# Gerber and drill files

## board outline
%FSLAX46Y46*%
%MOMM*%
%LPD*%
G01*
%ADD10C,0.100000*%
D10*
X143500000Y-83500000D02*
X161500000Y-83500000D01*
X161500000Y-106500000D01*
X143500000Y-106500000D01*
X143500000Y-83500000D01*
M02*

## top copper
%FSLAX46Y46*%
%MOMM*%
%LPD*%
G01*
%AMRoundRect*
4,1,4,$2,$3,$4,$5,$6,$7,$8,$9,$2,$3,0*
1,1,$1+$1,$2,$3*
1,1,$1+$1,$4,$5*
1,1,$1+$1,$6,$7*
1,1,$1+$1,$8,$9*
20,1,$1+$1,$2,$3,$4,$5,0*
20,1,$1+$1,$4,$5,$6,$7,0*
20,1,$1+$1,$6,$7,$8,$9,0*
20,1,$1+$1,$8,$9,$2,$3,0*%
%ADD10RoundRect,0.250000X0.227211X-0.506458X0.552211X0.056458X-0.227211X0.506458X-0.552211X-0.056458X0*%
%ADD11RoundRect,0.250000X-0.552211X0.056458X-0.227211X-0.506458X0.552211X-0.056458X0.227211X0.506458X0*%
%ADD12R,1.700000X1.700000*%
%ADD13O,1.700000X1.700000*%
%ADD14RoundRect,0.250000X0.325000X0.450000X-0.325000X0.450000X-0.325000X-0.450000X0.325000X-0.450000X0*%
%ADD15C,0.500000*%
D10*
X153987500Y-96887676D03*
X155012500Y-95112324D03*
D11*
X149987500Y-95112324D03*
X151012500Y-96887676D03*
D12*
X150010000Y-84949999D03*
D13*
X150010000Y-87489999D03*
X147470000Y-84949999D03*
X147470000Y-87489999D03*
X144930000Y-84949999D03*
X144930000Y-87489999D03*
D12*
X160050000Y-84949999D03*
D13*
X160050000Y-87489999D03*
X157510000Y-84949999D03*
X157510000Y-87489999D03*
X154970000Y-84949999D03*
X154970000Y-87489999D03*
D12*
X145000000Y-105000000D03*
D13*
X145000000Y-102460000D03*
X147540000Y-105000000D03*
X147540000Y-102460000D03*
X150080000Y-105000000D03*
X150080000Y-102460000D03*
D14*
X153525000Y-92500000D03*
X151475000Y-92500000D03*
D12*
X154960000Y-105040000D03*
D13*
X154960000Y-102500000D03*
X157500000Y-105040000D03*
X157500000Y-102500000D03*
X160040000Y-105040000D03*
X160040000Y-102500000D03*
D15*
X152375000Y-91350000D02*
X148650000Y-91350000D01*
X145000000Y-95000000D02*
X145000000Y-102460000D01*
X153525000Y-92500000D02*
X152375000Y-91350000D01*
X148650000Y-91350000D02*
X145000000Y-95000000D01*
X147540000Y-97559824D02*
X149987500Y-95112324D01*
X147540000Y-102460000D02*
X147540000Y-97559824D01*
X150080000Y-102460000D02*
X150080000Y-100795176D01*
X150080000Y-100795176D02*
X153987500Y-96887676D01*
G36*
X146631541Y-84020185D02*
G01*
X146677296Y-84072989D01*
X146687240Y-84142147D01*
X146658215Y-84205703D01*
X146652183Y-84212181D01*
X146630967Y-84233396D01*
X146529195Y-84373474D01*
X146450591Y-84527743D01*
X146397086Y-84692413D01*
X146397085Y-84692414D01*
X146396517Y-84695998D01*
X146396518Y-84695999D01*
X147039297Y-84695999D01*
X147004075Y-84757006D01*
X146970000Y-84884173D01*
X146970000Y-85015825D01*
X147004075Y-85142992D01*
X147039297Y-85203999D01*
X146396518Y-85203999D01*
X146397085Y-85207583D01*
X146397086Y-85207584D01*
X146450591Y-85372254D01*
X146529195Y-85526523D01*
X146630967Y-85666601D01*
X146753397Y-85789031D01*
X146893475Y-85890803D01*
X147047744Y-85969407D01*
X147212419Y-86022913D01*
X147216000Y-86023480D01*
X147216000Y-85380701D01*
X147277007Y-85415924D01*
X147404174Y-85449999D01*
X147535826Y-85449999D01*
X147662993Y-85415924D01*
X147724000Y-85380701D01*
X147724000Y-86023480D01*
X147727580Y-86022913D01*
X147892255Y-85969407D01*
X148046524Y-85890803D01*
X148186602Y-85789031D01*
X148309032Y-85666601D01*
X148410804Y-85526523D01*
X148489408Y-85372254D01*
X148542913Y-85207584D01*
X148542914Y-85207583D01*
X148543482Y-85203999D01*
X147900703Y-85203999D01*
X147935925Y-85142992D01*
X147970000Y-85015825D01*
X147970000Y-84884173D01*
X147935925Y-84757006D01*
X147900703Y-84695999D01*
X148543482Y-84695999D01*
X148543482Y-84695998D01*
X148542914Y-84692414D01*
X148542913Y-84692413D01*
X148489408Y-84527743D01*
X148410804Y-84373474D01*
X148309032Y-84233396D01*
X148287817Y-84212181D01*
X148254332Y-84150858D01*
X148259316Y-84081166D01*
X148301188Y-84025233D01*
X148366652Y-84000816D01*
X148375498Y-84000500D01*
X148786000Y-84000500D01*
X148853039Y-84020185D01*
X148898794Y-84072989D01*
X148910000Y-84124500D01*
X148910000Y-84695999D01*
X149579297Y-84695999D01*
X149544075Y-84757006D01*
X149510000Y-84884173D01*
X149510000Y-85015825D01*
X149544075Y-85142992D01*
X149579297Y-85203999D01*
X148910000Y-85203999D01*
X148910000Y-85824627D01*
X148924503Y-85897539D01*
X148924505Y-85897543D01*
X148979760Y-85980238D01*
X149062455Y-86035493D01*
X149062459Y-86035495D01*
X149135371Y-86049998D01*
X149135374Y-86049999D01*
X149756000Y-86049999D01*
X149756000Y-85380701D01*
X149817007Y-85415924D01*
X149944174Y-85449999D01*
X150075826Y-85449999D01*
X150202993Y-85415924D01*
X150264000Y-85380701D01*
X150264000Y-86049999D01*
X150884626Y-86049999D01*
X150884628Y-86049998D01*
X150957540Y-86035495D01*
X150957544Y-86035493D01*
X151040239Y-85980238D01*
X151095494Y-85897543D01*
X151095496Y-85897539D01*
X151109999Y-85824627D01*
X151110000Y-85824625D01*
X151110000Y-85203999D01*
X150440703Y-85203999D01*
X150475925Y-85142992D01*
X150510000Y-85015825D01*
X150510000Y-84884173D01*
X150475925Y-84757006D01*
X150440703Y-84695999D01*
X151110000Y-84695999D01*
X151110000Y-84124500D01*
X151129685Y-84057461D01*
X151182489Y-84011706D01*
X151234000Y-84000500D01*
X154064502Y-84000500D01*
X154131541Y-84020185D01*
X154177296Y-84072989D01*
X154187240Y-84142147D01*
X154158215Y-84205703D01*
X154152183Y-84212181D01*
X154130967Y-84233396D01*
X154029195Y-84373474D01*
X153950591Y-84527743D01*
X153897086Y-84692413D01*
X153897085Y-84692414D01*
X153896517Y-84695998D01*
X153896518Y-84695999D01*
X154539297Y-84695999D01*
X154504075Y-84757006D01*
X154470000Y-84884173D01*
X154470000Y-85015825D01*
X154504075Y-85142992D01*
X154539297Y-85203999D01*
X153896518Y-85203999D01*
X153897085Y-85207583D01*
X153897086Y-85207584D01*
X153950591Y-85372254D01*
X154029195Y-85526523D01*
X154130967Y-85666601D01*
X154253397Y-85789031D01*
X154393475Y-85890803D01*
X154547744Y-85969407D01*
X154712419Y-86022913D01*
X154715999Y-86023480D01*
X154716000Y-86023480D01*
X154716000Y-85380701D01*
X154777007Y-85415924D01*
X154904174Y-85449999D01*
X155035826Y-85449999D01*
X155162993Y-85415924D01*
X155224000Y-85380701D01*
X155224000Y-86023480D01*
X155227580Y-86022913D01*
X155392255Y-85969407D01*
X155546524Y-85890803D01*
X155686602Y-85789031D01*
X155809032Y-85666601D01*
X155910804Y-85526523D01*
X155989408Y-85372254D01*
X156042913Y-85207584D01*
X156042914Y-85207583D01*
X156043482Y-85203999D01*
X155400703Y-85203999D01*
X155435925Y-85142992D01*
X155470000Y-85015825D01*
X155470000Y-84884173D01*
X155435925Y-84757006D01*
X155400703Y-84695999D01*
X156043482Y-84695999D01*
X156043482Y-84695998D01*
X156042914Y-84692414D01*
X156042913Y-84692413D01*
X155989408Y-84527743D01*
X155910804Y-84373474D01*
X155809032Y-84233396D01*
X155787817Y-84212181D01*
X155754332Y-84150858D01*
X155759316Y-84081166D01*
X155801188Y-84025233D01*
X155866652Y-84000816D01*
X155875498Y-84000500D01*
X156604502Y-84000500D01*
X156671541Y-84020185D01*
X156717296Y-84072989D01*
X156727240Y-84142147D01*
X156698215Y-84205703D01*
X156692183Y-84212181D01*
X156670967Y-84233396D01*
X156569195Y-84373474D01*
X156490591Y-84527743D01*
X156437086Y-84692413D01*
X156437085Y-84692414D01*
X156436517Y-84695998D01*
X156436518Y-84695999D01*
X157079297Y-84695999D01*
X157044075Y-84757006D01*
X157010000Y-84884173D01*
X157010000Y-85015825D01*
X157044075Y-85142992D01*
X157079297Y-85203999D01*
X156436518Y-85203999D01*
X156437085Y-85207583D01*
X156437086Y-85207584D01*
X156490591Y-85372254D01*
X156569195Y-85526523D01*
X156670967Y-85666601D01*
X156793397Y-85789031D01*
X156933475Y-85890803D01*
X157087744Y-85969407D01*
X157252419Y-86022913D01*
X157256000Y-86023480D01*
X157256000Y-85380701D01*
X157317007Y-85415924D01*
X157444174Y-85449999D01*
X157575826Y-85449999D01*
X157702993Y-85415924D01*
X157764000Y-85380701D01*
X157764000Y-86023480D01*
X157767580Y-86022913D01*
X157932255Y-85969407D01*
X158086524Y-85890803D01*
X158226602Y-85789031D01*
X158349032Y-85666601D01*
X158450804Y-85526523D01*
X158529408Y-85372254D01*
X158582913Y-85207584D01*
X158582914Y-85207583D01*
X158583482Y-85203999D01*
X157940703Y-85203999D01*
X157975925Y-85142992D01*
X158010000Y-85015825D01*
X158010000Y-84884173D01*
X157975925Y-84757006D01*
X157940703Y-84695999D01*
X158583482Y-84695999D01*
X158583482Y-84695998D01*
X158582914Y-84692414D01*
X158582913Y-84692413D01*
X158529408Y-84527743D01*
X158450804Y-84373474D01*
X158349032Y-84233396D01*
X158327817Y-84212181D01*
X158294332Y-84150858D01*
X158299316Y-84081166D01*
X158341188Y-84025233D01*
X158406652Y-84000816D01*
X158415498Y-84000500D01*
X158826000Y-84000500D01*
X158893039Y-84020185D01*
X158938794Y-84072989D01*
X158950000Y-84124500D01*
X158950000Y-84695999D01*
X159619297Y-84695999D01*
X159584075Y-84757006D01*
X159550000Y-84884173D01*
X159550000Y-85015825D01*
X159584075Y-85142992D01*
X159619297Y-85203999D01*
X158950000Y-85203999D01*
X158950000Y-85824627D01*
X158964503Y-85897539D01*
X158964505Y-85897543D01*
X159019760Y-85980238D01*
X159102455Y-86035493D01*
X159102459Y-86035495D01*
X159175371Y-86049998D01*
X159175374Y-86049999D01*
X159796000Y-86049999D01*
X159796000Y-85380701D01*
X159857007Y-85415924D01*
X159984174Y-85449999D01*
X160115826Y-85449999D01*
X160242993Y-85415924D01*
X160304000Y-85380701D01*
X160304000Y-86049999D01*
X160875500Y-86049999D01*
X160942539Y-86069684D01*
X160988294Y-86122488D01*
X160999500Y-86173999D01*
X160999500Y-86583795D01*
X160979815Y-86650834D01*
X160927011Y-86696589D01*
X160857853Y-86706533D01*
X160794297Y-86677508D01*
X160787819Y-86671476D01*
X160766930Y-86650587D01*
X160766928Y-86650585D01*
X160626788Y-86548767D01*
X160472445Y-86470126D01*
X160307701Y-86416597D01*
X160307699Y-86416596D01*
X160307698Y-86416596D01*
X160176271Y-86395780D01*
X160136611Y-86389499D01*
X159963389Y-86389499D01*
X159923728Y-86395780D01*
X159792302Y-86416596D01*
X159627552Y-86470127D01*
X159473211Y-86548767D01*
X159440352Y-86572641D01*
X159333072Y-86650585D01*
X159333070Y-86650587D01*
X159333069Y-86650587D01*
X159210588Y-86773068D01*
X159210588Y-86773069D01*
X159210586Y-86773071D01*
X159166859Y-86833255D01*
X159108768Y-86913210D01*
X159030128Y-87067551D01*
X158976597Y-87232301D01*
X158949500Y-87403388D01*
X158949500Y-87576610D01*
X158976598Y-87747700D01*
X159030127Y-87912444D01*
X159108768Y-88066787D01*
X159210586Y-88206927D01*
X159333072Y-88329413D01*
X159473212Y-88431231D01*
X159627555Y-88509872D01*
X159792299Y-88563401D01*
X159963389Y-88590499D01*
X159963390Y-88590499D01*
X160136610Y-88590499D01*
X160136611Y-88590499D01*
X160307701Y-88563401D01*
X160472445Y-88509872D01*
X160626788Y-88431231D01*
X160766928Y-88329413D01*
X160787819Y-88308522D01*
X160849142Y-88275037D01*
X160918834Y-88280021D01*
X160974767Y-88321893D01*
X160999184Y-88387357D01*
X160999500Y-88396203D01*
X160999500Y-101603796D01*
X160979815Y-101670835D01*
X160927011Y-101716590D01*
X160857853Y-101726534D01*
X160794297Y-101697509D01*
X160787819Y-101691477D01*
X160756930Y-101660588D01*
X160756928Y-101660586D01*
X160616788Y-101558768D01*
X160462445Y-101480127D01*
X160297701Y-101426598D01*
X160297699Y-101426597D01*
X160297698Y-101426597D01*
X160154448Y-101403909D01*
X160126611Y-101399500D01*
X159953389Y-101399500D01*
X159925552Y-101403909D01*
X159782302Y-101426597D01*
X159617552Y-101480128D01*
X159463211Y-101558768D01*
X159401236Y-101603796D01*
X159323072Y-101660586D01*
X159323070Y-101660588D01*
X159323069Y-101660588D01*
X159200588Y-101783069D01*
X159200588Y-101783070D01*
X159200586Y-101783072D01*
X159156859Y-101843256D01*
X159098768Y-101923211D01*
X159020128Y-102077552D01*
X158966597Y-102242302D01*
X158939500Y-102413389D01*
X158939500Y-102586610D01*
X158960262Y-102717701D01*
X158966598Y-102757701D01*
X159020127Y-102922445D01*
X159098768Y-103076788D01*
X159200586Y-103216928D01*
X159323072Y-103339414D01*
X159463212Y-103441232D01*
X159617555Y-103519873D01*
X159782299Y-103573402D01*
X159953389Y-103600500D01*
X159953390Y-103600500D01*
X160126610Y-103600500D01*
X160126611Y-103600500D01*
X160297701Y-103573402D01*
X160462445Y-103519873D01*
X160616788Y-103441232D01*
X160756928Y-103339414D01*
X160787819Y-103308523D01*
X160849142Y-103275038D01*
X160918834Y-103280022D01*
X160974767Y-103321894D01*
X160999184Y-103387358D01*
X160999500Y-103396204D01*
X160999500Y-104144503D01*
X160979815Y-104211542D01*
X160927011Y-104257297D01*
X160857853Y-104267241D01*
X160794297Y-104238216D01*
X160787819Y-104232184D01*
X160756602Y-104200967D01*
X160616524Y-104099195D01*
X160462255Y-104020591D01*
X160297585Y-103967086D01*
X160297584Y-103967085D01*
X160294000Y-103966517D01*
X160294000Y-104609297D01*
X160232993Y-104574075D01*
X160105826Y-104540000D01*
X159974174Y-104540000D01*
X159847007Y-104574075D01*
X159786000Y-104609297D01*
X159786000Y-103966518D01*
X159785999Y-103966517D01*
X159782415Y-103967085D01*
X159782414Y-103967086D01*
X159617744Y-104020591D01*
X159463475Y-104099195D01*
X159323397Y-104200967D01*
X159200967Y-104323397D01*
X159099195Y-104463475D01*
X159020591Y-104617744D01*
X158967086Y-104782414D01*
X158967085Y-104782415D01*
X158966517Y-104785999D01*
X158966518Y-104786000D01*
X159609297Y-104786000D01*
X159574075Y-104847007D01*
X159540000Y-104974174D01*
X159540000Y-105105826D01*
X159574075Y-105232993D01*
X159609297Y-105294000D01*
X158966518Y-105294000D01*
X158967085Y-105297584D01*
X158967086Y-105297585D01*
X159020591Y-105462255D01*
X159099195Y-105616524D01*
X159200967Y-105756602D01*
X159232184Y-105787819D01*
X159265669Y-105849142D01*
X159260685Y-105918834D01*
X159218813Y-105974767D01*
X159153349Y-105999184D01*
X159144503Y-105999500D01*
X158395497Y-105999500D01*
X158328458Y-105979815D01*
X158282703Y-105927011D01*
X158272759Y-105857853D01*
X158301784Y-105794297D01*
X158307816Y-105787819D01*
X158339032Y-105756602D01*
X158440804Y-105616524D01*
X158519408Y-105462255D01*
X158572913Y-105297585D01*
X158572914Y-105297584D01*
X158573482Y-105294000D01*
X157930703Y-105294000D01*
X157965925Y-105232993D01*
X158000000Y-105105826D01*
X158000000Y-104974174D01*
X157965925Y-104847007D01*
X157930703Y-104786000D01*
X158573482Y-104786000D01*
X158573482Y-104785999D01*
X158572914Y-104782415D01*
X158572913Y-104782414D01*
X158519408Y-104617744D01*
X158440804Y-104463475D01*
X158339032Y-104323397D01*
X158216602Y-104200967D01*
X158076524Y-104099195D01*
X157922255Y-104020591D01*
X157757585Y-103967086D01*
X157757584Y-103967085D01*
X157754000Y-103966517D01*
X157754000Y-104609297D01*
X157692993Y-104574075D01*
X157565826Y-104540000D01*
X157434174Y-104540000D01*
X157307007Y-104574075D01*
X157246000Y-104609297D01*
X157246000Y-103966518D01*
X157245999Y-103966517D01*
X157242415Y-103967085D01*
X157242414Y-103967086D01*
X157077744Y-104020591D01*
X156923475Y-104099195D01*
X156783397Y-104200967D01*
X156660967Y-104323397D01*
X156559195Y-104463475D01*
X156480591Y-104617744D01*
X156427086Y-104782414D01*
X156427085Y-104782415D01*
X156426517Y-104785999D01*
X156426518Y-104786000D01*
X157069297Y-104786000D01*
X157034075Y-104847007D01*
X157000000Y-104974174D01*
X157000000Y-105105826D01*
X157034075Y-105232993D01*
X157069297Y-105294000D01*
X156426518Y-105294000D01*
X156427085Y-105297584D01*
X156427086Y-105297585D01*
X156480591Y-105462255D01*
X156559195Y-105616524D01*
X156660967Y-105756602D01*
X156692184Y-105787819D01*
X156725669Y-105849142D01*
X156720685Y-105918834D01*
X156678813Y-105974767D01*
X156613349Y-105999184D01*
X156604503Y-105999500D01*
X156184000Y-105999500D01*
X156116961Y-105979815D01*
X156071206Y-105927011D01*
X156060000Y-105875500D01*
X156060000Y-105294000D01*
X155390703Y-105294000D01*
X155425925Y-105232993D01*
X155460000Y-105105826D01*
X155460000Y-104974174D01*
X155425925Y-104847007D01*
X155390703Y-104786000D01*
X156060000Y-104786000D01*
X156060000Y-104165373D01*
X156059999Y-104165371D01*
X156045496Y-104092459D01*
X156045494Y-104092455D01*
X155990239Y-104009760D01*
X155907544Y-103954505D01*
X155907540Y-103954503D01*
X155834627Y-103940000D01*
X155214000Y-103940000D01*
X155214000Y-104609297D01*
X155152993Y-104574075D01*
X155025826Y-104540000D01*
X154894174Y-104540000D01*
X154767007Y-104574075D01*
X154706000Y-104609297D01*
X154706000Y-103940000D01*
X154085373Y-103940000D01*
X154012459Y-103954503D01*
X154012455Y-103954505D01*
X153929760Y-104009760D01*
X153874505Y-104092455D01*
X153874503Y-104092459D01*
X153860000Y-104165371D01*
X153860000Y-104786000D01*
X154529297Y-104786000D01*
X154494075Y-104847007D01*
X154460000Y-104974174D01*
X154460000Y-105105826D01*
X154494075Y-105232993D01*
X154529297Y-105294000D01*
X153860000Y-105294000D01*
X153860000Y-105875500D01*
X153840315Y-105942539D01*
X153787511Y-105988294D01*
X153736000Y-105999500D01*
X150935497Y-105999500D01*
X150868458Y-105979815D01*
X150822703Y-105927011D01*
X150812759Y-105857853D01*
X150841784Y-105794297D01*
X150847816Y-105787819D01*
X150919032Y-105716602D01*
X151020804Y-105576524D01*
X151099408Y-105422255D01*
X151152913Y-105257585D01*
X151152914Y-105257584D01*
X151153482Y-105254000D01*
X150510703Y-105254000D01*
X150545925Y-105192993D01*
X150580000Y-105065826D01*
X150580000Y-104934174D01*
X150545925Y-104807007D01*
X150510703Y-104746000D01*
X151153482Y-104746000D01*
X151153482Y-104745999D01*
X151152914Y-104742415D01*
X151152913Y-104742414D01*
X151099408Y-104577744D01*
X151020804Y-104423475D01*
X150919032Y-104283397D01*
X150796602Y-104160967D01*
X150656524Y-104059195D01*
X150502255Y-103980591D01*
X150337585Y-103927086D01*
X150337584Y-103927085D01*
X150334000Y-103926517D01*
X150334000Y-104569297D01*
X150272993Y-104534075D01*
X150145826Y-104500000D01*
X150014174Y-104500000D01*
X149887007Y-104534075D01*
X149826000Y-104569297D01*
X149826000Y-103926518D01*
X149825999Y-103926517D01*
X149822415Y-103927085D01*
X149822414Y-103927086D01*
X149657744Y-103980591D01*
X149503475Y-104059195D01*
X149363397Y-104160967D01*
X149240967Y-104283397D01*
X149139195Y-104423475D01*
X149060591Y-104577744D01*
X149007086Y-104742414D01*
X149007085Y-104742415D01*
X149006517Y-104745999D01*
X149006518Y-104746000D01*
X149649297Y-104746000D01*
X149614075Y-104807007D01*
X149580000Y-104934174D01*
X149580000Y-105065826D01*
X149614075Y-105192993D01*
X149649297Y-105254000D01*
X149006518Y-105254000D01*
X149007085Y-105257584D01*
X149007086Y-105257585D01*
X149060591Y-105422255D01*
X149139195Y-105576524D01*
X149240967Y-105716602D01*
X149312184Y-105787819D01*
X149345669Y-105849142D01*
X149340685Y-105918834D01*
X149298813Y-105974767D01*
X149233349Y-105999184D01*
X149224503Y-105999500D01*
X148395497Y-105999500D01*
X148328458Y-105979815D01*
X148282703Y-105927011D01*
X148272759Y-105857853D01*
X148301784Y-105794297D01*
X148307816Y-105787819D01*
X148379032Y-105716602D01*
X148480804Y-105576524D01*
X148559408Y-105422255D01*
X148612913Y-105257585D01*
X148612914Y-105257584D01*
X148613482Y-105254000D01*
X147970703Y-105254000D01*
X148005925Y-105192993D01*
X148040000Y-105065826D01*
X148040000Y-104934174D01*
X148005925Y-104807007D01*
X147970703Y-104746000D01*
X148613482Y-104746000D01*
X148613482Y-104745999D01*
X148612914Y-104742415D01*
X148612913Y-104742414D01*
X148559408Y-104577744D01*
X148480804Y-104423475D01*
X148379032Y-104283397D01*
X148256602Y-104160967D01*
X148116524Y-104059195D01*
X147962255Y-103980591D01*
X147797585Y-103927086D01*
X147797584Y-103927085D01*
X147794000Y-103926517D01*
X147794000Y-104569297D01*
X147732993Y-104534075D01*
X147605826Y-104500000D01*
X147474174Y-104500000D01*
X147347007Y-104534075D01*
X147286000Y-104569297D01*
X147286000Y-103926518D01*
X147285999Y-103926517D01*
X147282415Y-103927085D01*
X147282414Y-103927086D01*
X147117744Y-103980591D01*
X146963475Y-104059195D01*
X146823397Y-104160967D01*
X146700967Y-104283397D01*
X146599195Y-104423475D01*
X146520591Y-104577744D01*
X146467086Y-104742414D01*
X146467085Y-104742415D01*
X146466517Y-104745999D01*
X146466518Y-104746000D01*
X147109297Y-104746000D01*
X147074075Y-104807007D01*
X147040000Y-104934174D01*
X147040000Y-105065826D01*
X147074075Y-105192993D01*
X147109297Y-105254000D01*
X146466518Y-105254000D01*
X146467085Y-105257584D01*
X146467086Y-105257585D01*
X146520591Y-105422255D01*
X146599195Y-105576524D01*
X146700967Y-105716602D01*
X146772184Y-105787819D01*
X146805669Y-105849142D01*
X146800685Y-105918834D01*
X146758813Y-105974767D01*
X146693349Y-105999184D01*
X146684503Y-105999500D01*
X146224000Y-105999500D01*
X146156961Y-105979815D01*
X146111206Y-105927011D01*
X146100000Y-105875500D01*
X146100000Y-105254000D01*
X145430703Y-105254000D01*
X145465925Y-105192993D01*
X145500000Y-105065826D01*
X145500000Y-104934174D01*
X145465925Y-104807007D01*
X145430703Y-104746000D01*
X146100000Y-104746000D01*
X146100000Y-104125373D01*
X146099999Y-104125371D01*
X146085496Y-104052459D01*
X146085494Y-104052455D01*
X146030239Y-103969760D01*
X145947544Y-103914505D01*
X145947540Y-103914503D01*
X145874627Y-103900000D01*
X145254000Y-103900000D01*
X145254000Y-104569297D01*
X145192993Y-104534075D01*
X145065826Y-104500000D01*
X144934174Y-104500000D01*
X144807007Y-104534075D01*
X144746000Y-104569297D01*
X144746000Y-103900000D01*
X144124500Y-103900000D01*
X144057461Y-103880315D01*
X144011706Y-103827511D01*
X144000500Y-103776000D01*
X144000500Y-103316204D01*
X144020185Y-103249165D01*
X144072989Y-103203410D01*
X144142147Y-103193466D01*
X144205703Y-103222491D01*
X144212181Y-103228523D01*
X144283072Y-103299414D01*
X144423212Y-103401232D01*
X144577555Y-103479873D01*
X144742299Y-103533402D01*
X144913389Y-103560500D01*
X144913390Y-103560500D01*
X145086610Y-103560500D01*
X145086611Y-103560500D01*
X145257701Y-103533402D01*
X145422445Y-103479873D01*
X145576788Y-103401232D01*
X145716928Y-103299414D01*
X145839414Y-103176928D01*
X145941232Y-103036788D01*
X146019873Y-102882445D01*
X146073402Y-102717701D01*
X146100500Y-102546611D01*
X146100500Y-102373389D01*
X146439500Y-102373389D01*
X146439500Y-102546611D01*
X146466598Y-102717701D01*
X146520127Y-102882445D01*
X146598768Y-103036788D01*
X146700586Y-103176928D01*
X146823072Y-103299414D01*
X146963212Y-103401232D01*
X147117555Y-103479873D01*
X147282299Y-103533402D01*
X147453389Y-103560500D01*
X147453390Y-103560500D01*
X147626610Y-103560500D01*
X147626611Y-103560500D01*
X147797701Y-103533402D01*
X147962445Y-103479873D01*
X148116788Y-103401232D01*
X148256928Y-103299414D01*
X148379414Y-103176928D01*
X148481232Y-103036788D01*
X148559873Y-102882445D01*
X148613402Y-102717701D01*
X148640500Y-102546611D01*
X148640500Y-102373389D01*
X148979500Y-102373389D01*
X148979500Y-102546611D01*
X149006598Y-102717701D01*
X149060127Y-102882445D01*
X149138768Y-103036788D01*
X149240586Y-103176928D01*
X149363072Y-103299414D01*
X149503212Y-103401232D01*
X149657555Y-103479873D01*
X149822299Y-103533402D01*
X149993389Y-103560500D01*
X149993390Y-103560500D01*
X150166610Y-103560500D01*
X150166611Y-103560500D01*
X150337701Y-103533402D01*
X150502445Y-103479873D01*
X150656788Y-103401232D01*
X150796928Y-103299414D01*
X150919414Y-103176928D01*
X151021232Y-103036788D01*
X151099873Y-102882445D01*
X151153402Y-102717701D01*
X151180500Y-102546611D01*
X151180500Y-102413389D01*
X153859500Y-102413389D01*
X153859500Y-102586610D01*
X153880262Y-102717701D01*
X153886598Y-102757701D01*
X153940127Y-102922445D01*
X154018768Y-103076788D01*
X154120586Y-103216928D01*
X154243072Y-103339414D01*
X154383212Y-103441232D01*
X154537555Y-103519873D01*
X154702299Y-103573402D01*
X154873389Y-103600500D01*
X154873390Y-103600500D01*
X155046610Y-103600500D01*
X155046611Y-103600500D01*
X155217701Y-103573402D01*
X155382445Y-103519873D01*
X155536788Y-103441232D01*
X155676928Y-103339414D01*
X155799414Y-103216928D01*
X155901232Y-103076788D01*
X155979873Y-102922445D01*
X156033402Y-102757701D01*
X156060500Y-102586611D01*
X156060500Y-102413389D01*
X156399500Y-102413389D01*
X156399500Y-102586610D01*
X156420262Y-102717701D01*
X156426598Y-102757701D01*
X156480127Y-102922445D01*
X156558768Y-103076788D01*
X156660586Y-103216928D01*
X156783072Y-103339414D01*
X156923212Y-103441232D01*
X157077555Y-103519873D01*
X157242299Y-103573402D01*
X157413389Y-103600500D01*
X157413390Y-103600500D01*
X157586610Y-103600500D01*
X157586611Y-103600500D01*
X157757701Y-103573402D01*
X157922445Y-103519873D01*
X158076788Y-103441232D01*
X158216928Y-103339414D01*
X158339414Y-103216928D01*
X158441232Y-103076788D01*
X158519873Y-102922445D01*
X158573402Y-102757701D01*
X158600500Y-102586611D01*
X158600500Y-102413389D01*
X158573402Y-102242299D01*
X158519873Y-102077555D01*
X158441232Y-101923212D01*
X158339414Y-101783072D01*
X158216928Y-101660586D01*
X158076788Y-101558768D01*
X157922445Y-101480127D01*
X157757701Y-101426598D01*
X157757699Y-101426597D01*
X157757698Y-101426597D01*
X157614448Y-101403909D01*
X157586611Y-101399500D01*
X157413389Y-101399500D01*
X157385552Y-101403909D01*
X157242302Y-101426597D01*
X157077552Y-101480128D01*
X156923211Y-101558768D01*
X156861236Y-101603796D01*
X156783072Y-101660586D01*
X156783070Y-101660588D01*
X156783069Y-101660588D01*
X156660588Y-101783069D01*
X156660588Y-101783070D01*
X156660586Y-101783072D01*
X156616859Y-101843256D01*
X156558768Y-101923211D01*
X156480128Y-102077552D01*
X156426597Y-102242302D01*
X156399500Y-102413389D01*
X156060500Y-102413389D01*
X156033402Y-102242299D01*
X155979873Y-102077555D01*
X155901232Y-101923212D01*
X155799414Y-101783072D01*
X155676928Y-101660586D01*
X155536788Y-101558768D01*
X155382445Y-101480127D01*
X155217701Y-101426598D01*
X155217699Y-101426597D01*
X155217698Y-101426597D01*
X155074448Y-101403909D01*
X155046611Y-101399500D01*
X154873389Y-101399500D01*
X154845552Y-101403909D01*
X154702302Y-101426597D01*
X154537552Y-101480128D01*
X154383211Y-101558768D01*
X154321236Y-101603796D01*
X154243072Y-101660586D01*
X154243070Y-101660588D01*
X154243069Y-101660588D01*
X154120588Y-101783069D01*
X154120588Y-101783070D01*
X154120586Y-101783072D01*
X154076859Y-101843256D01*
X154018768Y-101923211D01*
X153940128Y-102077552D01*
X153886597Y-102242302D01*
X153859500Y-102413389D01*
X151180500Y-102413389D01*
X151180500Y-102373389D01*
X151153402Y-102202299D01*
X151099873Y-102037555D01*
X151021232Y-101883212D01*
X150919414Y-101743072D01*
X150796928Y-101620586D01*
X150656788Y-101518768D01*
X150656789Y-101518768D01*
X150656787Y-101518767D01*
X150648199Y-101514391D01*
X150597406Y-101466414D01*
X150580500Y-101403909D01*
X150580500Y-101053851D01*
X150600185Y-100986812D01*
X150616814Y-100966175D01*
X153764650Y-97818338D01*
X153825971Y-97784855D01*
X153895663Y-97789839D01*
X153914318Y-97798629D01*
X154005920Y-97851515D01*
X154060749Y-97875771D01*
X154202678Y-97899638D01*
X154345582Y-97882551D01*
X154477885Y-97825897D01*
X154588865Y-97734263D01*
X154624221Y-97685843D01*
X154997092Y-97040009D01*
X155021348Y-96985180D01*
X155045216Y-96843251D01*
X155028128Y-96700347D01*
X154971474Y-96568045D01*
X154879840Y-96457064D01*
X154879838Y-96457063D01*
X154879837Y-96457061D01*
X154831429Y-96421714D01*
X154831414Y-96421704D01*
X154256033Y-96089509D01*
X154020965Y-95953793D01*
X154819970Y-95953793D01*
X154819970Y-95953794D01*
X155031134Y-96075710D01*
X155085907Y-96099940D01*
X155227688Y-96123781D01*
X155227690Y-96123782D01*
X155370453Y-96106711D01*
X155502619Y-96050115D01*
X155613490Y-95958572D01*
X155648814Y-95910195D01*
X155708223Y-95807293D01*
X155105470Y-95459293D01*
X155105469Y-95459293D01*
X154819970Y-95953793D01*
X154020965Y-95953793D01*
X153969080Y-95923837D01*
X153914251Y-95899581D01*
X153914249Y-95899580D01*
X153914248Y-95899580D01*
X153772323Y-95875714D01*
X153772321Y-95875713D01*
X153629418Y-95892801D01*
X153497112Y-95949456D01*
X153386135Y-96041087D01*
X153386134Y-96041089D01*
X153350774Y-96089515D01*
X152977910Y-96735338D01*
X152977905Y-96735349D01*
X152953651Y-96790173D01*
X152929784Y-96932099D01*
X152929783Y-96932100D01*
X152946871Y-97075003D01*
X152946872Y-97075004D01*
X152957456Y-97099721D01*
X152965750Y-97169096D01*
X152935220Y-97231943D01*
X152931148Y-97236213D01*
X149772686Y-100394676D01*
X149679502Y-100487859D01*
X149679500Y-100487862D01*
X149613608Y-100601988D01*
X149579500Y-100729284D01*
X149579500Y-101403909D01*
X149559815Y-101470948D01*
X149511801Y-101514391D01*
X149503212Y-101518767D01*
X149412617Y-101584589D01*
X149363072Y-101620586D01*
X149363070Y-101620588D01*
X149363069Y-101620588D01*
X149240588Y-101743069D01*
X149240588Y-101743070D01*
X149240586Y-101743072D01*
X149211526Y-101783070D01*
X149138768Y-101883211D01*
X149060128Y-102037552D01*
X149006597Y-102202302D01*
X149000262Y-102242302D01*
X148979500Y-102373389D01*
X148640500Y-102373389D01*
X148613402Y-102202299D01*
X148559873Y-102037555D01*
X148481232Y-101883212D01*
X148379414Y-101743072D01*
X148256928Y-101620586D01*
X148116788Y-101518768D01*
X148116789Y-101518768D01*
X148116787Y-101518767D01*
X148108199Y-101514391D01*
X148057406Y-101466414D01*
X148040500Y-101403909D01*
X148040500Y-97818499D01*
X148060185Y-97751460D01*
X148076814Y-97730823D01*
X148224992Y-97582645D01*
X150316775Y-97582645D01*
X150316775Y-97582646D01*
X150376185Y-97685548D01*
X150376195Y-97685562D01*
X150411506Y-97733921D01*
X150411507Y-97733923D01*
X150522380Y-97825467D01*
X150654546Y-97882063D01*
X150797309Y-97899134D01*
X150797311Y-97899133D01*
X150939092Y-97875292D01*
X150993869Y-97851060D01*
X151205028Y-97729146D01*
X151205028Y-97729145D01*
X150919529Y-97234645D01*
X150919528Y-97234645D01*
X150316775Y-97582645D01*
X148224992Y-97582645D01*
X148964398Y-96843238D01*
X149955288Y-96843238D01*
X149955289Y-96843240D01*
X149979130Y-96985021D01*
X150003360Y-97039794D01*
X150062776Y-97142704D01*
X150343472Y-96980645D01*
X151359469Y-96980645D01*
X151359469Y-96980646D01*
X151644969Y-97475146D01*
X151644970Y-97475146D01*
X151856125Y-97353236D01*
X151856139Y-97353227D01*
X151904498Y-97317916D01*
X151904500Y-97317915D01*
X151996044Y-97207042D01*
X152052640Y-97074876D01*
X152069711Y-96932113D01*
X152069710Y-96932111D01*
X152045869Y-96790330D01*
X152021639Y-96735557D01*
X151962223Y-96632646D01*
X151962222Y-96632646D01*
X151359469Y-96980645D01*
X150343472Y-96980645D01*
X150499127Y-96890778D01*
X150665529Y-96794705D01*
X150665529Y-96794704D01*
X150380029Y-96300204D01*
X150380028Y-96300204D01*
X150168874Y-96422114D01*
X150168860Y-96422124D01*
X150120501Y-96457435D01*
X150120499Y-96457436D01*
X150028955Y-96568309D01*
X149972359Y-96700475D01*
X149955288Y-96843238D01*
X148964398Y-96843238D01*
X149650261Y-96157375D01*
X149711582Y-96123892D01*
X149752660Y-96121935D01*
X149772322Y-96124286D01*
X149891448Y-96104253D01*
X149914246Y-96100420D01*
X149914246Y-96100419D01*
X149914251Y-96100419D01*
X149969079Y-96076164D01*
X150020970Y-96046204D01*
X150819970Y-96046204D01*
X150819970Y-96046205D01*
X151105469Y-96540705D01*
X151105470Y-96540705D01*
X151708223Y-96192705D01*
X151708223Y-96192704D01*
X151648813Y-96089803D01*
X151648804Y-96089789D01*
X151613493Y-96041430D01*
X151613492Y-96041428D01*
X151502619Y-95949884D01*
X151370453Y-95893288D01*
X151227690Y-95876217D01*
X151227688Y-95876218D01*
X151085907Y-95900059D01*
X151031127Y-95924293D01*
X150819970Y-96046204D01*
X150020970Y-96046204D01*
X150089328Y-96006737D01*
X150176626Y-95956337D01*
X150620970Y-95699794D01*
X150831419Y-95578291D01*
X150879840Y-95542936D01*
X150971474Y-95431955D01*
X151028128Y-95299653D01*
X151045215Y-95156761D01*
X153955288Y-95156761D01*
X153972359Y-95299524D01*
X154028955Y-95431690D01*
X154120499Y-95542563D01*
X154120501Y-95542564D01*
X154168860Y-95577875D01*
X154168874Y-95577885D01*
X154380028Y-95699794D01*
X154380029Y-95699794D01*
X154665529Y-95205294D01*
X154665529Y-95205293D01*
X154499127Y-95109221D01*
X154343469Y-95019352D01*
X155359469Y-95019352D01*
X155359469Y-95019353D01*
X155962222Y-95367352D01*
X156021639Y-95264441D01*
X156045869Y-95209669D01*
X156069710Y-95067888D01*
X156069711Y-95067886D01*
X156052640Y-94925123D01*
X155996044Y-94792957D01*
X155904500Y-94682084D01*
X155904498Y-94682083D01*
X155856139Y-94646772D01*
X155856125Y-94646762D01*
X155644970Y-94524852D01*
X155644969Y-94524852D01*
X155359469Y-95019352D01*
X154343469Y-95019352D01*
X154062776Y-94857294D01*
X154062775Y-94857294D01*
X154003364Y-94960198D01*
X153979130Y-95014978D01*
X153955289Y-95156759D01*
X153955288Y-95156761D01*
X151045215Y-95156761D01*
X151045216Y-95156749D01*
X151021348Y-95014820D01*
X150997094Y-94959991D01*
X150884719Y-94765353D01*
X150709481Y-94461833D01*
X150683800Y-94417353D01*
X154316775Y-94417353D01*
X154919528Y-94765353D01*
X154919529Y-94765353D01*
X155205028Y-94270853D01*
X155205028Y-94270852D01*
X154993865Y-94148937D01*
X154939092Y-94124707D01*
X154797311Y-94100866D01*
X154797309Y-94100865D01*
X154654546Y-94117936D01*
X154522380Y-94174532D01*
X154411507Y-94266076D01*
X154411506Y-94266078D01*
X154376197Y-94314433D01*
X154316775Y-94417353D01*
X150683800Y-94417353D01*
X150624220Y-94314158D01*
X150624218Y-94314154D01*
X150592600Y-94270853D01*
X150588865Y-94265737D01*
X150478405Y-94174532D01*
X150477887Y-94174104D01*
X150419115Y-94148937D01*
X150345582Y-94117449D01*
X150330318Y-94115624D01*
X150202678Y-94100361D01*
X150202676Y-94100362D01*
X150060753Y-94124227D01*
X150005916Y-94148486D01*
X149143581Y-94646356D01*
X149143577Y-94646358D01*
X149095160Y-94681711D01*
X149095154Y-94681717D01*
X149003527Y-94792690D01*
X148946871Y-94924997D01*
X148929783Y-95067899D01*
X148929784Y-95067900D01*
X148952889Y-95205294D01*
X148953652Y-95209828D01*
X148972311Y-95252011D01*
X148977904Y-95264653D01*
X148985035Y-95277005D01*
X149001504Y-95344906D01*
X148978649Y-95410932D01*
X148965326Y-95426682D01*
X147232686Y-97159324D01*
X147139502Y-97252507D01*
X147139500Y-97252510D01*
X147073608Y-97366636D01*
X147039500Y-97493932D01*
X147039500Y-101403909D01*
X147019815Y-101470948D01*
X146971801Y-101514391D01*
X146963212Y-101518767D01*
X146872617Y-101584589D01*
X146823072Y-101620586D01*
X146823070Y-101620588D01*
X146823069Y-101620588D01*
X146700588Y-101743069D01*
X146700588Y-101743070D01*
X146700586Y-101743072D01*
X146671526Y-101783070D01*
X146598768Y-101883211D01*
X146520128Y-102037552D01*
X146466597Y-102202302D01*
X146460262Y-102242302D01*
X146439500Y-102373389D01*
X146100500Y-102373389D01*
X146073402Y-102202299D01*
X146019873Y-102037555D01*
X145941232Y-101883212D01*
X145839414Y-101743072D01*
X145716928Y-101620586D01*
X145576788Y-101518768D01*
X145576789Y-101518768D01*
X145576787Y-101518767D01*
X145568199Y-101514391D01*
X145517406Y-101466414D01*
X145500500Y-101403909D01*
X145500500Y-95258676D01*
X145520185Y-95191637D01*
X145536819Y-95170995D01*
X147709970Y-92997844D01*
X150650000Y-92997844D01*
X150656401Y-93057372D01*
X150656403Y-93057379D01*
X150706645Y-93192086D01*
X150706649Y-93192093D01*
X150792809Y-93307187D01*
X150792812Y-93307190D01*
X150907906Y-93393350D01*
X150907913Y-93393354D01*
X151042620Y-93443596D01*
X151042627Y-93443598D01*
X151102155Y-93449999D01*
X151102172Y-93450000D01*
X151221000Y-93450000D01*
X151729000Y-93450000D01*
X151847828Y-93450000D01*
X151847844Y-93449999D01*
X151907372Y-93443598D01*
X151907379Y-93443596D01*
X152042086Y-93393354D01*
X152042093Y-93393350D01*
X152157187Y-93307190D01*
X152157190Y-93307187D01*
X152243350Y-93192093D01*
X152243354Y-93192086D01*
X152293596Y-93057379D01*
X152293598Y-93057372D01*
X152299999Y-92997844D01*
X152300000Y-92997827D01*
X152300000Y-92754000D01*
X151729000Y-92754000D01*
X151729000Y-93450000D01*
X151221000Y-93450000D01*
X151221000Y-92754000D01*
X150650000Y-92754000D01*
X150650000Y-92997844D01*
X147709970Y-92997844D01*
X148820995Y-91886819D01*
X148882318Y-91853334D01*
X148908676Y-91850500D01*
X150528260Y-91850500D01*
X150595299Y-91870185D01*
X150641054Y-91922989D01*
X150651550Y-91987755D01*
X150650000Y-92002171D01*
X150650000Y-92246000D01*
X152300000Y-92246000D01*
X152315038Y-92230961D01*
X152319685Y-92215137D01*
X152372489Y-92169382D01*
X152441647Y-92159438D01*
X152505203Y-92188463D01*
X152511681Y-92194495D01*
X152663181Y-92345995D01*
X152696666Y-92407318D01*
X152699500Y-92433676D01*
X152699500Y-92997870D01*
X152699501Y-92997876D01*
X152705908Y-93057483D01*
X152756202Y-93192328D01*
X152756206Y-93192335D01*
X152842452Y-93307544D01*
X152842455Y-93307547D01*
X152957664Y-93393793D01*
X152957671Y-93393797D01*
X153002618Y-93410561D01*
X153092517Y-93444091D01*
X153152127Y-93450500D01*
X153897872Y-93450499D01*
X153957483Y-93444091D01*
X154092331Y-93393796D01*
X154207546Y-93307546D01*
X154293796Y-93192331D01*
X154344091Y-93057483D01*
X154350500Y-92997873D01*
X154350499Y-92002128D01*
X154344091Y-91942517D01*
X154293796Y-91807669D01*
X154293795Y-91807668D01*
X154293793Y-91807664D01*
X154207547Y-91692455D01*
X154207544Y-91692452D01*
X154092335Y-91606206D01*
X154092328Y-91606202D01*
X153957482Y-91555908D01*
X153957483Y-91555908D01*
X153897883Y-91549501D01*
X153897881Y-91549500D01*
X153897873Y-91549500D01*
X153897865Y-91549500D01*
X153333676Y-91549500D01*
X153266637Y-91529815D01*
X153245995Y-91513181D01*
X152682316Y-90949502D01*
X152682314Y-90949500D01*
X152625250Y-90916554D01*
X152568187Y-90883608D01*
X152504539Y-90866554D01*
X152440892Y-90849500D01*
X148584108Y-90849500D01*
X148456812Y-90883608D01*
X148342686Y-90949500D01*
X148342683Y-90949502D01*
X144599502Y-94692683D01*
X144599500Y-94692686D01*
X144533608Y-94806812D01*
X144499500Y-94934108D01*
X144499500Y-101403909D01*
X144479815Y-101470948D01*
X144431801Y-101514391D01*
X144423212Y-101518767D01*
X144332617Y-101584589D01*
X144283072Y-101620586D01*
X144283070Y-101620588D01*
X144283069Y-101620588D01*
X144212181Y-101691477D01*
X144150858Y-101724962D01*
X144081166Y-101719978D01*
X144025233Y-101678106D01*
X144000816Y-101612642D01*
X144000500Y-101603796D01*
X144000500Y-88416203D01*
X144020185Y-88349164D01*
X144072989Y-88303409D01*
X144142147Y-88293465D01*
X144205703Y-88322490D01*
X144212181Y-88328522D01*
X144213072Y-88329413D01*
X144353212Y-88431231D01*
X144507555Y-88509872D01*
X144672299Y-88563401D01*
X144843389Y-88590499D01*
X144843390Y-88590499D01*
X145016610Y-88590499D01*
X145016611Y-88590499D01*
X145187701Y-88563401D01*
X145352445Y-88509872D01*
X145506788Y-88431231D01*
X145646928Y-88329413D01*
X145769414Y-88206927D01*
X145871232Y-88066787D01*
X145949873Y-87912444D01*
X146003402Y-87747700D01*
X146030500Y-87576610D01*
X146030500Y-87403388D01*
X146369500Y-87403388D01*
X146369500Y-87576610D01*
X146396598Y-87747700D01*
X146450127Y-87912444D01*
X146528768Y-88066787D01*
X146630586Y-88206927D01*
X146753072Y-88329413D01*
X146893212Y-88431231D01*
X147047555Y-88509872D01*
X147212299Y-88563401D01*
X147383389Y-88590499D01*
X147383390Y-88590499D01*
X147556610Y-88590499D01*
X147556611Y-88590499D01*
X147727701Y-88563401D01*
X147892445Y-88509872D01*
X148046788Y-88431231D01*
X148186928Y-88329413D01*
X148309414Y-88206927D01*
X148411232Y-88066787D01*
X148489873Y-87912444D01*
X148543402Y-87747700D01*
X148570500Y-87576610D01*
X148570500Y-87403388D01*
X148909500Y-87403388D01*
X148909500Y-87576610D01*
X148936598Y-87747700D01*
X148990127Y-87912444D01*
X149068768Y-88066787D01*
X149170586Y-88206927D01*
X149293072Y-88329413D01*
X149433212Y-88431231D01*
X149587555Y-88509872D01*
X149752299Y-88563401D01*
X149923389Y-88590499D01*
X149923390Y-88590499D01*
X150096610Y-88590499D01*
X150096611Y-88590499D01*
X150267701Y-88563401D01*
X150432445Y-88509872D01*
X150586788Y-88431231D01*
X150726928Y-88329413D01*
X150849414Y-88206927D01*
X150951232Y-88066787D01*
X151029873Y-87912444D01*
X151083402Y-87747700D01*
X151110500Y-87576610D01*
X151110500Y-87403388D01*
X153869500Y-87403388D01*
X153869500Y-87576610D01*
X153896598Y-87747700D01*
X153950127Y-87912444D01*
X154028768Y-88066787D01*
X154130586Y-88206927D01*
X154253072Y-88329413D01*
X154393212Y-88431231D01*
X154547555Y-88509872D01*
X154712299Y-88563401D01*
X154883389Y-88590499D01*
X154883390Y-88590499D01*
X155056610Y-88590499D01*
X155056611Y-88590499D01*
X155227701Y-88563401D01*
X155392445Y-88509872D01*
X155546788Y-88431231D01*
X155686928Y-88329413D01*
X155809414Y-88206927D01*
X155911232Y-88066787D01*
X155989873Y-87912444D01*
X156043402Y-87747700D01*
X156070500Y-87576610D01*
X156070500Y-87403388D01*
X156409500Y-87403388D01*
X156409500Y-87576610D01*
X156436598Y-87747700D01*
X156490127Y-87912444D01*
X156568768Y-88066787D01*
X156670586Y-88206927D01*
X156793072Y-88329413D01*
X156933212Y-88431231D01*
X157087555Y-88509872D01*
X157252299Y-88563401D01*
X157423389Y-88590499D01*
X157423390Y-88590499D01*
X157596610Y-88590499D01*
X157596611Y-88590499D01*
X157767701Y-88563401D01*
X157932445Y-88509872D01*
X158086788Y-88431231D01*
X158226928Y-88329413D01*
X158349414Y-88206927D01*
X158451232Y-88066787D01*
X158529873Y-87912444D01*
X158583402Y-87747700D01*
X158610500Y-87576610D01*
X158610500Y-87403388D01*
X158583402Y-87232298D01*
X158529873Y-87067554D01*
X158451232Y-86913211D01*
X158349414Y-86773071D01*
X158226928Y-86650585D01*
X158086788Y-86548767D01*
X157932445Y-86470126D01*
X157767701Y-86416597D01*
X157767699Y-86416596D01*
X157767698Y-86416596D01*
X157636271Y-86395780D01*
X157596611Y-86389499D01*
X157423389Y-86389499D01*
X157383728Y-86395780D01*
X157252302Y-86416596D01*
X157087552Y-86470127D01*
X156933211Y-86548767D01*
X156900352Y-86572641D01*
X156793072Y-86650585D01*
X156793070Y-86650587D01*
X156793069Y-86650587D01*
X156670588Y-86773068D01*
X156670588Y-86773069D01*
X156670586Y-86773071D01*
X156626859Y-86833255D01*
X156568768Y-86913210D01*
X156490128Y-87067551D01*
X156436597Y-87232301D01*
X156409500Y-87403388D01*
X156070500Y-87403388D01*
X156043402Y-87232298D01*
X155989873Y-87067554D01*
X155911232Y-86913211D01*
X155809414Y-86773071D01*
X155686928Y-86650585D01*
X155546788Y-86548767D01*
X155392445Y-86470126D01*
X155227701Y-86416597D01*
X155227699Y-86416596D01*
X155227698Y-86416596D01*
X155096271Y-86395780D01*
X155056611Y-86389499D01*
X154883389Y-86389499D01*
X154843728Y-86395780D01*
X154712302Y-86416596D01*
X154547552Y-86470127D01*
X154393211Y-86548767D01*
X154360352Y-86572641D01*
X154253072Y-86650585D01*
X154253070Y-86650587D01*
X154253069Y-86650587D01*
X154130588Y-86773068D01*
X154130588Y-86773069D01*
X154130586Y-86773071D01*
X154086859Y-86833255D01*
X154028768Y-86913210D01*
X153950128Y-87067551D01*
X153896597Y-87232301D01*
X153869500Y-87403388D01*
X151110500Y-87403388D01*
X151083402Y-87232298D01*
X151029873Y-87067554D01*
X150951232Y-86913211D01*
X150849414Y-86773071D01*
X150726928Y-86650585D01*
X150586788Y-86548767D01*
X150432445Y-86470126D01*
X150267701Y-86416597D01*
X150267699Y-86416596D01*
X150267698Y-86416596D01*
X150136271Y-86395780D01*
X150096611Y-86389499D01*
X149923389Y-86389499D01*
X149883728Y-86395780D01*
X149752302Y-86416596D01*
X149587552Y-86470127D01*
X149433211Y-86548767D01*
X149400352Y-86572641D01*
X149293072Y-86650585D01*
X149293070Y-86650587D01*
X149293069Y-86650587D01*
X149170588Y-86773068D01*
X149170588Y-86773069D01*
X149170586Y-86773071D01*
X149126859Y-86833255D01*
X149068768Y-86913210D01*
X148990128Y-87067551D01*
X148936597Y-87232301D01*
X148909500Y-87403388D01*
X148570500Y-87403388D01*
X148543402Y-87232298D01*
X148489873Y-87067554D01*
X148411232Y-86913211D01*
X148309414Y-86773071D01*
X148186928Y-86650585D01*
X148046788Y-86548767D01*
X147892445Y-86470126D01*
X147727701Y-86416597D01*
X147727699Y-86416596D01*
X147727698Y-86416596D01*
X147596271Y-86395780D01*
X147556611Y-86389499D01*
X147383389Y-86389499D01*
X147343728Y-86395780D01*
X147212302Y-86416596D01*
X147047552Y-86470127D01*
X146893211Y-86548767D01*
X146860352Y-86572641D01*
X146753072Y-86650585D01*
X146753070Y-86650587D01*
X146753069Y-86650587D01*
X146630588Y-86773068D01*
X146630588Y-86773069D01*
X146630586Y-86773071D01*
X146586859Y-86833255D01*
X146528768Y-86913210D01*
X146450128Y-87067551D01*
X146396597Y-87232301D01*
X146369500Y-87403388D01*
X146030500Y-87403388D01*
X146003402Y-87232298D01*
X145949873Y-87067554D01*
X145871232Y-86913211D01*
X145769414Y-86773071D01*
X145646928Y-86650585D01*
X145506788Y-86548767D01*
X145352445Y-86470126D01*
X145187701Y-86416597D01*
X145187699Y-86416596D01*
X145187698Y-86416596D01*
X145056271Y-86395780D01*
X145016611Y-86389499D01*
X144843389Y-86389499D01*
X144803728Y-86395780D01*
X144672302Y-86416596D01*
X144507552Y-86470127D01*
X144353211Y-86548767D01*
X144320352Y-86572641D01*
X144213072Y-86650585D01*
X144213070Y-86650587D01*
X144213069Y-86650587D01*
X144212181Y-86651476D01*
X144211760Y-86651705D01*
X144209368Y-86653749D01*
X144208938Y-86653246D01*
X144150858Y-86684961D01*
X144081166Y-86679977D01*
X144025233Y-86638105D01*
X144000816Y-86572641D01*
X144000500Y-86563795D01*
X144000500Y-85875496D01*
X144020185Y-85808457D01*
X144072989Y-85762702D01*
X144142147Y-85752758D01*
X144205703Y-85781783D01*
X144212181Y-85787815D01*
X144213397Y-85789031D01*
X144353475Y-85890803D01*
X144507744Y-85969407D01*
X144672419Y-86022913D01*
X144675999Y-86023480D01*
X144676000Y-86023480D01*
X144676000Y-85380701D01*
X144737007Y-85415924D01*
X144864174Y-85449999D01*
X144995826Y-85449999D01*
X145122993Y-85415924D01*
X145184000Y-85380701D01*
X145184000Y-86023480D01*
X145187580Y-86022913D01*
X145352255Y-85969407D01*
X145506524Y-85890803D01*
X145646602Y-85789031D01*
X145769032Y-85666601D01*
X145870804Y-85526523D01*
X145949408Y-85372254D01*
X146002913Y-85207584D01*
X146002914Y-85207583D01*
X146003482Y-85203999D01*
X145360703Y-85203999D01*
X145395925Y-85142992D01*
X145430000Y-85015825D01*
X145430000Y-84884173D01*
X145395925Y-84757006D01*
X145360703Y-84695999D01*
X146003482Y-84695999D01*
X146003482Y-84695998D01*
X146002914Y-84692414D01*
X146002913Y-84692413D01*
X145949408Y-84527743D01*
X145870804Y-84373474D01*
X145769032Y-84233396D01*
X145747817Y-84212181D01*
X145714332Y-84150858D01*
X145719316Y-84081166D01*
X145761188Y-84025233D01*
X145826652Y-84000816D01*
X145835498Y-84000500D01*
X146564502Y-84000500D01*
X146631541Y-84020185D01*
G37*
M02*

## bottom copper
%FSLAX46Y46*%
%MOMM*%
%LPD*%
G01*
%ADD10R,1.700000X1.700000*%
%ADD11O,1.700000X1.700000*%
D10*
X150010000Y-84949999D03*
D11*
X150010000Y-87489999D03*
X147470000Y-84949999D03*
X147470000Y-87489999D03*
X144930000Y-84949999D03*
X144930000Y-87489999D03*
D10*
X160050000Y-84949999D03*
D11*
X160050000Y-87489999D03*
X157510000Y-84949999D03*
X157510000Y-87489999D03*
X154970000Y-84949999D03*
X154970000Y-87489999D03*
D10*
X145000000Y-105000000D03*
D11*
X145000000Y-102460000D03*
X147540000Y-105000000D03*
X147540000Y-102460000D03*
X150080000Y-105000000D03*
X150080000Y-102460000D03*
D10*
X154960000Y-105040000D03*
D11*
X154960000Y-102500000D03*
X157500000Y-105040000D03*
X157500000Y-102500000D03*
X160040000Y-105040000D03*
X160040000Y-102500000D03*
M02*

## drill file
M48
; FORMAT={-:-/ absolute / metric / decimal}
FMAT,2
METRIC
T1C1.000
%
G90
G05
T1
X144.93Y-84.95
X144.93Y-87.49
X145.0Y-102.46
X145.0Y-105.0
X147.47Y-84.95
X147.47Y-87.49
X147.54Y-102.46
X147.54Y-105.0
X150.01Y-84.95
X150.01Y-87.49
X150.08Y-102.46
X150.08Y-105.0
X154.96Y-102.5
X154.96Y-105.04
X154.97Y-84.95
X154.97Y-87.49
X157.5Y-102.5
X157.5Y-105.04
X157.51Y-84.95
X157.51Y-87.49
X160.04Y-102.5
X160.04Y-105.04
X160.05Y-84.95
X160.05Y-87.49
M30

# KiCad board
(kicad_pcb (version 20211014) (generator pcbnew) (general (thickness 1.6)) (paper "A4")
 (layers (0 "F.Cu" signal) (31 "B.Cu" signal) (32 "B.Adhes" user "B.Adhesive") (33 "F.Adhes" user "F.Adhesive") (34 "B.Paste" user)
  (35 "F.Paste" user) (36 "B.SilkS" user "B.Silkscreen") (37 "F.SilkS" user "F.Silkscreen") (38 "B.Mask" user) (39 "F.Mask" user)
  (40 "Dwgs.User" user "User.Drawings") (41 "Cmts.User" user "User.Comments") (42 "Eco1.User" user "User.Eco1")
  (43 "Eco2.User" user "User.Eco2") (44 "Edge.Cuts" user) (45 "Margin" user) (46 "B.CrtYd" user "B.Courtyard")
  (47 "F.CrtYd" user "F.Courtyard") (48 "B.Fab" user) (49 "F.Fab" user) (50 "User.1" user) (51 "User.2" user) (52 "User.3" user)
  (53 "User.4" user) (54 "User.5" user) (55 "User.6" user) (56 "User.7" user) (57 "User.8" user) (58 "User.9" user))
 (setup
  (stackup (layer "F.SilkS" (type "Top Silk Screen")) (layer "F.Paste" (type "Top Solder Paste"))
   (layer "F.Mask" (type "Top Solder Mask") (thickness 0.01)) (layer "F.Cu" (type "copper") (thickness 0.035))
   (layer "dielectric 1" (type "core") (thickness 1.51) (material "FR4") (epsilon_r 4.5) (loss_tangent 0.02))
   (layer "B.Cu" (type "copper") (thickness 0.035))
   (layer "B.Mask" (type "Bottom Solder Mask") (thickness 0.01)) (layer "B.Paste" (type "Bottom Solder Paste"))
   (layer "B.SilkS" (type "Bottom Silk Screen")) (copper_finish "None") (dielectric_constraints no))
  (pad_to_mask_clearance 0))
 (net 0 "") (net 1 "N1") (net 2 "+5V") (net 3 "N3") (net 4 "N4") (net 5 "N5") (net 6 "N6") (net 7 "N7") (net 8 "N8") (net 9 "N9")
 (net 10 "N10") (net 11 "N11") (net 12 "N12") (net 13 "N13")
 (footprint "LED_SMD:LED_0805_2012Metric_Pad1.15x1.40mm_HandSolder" (layer "F.Cu") (at 154.5 96 60)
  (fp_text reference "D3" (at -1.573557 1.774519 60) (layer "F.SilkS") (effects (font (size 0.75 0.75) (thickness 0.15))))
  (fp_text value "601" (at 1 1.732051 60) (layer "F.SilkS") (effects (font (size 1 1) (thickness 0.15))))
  (pad "1" smd roundrect (at -1.025 0 60) (size 1.15 1.4) (layers "F.Cu" "F.Paste" "F.Mask") (roundrect_rratio 0.217391) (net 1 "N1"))
  (pad "2" smd roundrect (at 1.025 0 60) (size 1.15 1.4) (layers "F.Cu" "F.Paste" "F.Mask") (roundrect_rratio 0.217391) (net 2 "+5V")))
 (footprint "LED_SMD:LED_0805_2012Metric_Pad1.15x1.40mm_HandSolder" (layer "F.Cu") (at 150.5 96 -60)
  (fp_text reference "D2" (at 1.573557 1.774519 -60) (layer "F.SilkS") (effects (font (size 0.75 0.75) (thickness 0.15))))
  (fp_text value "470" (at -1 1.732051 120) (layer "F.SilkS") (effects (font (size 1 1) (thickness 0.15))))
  (pad "1" smd roundrect (at -1.025 0 300) (size 1.15 1.4) (layers "F.Cu" "F.Paste" "F.Mask") (roundrect_rratio 0.217391) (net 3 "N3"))
  (pad "2" smd roundrect (at 1.025 0 300) (size 1.15 1.4) (layers "F.Cu" "F.Paste" "F.Mask") (roundrect_rratio 0.217391) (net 2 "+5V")))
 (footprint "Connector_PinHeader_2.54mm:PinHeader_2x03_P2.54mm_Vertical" (layer "F.Cu") (at 150.01 84.949999 -90)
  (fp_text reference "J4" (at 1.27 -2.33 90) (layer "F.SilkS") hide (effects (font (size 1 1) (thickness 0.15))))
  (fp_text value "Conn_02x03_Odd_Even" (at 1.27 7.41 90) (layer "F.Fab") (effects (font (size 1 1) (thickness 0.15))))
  (pad "1" thru_hole rect (at 0 0 270) (size 1.7 1.7) (drill 1) (layers *.Cu *.Mask) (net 2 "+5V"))
  (pad "2" thru_hole oval (at 2.54 0 270) (size 1.7 1.7) (drill 1) (layers *.Cu *.Mask) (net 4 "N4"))
  (pad "3" thru_hole oval (at 0 2.54 270) (size 1.7 1.7) (drill 1) (layers *.Cu *.Mask) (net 2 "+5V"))
  (pad "4" thru_hole oval (at 2.54 2.54 270) (size 1.7 1.7) (drill 1) (layers *.Cu *.Mask) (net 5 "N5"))
  (pad "5" thru_hole oval (at 0 5.08 270) (size 1.7 1.7) (drill 1) (layers *.Cu *.Mask) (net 2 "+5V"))
  (pad "6" thru_hole oval (at 2.54 5.08 270) (size 1.7 1.7) (drill 1) (layers *.Cu *.Mask) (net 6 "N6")))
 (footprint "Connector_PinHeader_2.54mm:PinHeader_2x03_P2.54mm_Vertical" (layer "F.Cu") (at 160.05 84.949999 -90)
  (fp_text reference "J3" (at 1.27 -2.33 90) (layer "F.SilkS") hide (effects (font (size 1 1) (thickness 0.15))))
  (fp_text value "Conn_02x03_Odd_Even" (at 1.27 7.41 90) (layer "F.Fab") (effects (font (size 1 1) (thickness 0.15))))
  (pad "1" thru_hole rect (at 0 0 270) (size 1.7 1.7) (drill 1) (layers *.Cu *.Mask) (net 2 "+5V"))
  (pad "2" thru_hole oval (at 2.54 0 270) (size 1.7 1.7) (drill 1) (layers *.Cu *.Mask) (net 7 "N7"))
  (pad "3" thru_hole oval (at 0 2.54 270) (size 1.7 1.7) (drill 1) (layers *.Cu *.Mask) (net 2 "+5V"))
  (pad "4" thru_hole oval (at 2.54 2.54 270) (size 1.7 1.7) (drill 1) (layers *.Cu *.Mask) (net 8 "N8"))
  (pad "5" thru_hole oval (at 0 5.08 270) (size 1.7 1.7) (drill 1) (layers *.Cu *.Mask) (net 2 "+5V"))
  (pad "6" thru_hole oval (at 2.54 5.08 270) (size 1.7 1.7) (drill 1) (layers *.Cu *.Mask) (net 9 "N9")))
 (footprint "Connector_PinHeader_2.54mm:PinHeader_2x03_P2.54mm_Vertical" (layer "F.Cu") (at 145 105 90)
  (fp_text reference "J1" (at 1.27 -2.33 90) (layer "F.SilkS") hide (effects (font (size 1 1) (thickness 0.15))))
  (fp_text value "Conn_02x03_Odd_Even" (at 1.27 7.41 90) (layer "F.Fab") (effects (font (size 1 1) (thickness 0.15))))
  (pad "1" thru_hole rect (at 0 0 90) (size 1.7 1.7) (drill 1) (layers *.Cu *.Mask) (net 2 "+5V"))
  (pad "2" thru_hole oval (at 2.54 0 90) (size 1.7 1.7) (drill 1) (layers *.Cu *.Mask) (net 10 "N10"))
  (pad "3" thru_hole oval (at 0 2.54 90) (size 1.7 1.7) (drill 1) (layers *.Cu *.Mask) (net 2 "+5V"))
  (pad "4" thru_hole oval (at 2.54 2.54 90) (size 1.7 1.7) (drill 1) (layers *.Cu *.Mask) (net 3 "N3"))
  (pad "5" thru_hole oval (at 0 5.08 90) (size 1.7 1.7) (drill 1) (layers *.Cu *.Mask) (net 2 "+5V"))
  (pad "6" thru_hole oval (at 2.54 5.08 90) (size 1.7 1.7) (drill 1) (layers *.Cu *.Mask) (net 1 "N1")))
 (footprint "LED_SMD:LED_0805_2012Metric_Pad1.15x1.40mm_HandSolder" (layer "F.Cu") (at 152.5 92.5 180)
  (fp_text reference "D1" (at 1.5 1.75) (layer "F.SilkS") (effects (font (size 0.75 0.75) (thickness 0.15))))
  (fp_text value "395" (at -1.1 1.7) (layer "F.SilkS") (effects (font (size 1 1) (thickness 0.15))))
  (pad "1" smd roundrect (at -1.025 0 180) (size 1.15 1.4) (layers "F.Cu" "F.Paste" "F.Mask") (roundrect_rratio 0.217391) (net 10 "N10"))
  (pad "2" smd roundrect (at 1.025 0 180) (size 1.15 1.4) (layers "F.Cu" "F.Paste" "F.Mask") (roundrect_rratio 0.217391) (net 2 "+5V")))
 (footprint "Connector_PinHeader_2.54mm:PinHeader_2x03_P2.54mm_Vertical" (layer "F.Cu") (at 154.96 105.04 90)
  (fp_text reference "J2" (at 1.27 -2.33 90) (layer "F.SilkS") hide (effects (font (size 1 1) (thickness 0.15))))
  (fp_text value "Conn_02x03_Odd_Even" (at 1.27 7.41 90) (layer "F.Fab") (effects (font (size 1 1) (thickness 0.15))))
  (pad "1" thru_hole rect (at 0 0 90) (size 1.7 1.7) (drill 1) (layers *.Cu *.Mask) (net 2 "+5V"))
  (pad "2" thru_hole oval (at 2.54 0 90) (size 1.7 1.7) (drill 1) (layers *.Cu *.Mask) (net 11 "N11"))
  (pad "3" thru_hole oval (at 0 2.54 90) (size 1.7 1.7) (drill 1) (layers *.Cu *.Mask) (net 2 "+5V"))
  (pad "4" thru_hole oval (at 2.54 2.54 90) (size 1.7 1.7) (drill 1) (layers *.Cu *.Mask) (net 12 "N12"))
  (pad "5" thru_hole oval (at 0 5.08 90) (size 1.7 1.7) (drill 1) (layers *.Cu *.Mask) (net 2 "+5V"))
  (pad "6" thru_hole oval (at 2.54 5.08 90) (size 1.7 1.7) (drill 1) (layers *.Cu *.Mask) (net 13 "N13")))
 (gr_rect (start 143.5 83.5) (end 161.5 106.5) (layer "Edge.Cuts") (width 0.1) (fill none))
 (segment (start 152.375 91.35) (end 148.65 91.35) (width 0.5) (layer "F.Cu") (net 10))
 (segment (start 145 95) (end 145 102.46) (width 0.5) (layer "F.Cu") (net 10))
 (segment (start 153.525 92.5) (end 152.375 91.35) (width 0.5) (layer "F.Cu") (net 10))
 (segment (start 148.65 91.35) (end 145 95) (width 0.5) (layer "F.Cu") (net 10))
 (segment (start 147.54 97.559824) (end 149.9875 95.112324) (width 0.5) (layer "F.Cu") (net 3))
 (segment (start 147.54 102.46) (end 147.54 97.559824) (width 0.5) (layer "F.Cu") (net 3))
 (segment (start 150.08 102.46) (end 150.08 100.795176) (width 0.5) (layer "F.Cu") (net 1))
 (segment (start 150.08 100.795176) (end 153.9875 96.887676) (width 0.5) (layer "F.Cu") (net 1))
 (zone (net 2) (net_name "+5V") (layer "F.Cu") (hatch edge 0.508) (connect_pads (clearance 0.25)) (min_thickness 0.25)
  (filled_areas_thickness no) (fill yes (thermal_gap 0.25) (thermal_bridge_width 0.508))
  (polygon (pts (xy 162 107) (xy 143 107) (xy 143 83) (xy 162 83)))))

